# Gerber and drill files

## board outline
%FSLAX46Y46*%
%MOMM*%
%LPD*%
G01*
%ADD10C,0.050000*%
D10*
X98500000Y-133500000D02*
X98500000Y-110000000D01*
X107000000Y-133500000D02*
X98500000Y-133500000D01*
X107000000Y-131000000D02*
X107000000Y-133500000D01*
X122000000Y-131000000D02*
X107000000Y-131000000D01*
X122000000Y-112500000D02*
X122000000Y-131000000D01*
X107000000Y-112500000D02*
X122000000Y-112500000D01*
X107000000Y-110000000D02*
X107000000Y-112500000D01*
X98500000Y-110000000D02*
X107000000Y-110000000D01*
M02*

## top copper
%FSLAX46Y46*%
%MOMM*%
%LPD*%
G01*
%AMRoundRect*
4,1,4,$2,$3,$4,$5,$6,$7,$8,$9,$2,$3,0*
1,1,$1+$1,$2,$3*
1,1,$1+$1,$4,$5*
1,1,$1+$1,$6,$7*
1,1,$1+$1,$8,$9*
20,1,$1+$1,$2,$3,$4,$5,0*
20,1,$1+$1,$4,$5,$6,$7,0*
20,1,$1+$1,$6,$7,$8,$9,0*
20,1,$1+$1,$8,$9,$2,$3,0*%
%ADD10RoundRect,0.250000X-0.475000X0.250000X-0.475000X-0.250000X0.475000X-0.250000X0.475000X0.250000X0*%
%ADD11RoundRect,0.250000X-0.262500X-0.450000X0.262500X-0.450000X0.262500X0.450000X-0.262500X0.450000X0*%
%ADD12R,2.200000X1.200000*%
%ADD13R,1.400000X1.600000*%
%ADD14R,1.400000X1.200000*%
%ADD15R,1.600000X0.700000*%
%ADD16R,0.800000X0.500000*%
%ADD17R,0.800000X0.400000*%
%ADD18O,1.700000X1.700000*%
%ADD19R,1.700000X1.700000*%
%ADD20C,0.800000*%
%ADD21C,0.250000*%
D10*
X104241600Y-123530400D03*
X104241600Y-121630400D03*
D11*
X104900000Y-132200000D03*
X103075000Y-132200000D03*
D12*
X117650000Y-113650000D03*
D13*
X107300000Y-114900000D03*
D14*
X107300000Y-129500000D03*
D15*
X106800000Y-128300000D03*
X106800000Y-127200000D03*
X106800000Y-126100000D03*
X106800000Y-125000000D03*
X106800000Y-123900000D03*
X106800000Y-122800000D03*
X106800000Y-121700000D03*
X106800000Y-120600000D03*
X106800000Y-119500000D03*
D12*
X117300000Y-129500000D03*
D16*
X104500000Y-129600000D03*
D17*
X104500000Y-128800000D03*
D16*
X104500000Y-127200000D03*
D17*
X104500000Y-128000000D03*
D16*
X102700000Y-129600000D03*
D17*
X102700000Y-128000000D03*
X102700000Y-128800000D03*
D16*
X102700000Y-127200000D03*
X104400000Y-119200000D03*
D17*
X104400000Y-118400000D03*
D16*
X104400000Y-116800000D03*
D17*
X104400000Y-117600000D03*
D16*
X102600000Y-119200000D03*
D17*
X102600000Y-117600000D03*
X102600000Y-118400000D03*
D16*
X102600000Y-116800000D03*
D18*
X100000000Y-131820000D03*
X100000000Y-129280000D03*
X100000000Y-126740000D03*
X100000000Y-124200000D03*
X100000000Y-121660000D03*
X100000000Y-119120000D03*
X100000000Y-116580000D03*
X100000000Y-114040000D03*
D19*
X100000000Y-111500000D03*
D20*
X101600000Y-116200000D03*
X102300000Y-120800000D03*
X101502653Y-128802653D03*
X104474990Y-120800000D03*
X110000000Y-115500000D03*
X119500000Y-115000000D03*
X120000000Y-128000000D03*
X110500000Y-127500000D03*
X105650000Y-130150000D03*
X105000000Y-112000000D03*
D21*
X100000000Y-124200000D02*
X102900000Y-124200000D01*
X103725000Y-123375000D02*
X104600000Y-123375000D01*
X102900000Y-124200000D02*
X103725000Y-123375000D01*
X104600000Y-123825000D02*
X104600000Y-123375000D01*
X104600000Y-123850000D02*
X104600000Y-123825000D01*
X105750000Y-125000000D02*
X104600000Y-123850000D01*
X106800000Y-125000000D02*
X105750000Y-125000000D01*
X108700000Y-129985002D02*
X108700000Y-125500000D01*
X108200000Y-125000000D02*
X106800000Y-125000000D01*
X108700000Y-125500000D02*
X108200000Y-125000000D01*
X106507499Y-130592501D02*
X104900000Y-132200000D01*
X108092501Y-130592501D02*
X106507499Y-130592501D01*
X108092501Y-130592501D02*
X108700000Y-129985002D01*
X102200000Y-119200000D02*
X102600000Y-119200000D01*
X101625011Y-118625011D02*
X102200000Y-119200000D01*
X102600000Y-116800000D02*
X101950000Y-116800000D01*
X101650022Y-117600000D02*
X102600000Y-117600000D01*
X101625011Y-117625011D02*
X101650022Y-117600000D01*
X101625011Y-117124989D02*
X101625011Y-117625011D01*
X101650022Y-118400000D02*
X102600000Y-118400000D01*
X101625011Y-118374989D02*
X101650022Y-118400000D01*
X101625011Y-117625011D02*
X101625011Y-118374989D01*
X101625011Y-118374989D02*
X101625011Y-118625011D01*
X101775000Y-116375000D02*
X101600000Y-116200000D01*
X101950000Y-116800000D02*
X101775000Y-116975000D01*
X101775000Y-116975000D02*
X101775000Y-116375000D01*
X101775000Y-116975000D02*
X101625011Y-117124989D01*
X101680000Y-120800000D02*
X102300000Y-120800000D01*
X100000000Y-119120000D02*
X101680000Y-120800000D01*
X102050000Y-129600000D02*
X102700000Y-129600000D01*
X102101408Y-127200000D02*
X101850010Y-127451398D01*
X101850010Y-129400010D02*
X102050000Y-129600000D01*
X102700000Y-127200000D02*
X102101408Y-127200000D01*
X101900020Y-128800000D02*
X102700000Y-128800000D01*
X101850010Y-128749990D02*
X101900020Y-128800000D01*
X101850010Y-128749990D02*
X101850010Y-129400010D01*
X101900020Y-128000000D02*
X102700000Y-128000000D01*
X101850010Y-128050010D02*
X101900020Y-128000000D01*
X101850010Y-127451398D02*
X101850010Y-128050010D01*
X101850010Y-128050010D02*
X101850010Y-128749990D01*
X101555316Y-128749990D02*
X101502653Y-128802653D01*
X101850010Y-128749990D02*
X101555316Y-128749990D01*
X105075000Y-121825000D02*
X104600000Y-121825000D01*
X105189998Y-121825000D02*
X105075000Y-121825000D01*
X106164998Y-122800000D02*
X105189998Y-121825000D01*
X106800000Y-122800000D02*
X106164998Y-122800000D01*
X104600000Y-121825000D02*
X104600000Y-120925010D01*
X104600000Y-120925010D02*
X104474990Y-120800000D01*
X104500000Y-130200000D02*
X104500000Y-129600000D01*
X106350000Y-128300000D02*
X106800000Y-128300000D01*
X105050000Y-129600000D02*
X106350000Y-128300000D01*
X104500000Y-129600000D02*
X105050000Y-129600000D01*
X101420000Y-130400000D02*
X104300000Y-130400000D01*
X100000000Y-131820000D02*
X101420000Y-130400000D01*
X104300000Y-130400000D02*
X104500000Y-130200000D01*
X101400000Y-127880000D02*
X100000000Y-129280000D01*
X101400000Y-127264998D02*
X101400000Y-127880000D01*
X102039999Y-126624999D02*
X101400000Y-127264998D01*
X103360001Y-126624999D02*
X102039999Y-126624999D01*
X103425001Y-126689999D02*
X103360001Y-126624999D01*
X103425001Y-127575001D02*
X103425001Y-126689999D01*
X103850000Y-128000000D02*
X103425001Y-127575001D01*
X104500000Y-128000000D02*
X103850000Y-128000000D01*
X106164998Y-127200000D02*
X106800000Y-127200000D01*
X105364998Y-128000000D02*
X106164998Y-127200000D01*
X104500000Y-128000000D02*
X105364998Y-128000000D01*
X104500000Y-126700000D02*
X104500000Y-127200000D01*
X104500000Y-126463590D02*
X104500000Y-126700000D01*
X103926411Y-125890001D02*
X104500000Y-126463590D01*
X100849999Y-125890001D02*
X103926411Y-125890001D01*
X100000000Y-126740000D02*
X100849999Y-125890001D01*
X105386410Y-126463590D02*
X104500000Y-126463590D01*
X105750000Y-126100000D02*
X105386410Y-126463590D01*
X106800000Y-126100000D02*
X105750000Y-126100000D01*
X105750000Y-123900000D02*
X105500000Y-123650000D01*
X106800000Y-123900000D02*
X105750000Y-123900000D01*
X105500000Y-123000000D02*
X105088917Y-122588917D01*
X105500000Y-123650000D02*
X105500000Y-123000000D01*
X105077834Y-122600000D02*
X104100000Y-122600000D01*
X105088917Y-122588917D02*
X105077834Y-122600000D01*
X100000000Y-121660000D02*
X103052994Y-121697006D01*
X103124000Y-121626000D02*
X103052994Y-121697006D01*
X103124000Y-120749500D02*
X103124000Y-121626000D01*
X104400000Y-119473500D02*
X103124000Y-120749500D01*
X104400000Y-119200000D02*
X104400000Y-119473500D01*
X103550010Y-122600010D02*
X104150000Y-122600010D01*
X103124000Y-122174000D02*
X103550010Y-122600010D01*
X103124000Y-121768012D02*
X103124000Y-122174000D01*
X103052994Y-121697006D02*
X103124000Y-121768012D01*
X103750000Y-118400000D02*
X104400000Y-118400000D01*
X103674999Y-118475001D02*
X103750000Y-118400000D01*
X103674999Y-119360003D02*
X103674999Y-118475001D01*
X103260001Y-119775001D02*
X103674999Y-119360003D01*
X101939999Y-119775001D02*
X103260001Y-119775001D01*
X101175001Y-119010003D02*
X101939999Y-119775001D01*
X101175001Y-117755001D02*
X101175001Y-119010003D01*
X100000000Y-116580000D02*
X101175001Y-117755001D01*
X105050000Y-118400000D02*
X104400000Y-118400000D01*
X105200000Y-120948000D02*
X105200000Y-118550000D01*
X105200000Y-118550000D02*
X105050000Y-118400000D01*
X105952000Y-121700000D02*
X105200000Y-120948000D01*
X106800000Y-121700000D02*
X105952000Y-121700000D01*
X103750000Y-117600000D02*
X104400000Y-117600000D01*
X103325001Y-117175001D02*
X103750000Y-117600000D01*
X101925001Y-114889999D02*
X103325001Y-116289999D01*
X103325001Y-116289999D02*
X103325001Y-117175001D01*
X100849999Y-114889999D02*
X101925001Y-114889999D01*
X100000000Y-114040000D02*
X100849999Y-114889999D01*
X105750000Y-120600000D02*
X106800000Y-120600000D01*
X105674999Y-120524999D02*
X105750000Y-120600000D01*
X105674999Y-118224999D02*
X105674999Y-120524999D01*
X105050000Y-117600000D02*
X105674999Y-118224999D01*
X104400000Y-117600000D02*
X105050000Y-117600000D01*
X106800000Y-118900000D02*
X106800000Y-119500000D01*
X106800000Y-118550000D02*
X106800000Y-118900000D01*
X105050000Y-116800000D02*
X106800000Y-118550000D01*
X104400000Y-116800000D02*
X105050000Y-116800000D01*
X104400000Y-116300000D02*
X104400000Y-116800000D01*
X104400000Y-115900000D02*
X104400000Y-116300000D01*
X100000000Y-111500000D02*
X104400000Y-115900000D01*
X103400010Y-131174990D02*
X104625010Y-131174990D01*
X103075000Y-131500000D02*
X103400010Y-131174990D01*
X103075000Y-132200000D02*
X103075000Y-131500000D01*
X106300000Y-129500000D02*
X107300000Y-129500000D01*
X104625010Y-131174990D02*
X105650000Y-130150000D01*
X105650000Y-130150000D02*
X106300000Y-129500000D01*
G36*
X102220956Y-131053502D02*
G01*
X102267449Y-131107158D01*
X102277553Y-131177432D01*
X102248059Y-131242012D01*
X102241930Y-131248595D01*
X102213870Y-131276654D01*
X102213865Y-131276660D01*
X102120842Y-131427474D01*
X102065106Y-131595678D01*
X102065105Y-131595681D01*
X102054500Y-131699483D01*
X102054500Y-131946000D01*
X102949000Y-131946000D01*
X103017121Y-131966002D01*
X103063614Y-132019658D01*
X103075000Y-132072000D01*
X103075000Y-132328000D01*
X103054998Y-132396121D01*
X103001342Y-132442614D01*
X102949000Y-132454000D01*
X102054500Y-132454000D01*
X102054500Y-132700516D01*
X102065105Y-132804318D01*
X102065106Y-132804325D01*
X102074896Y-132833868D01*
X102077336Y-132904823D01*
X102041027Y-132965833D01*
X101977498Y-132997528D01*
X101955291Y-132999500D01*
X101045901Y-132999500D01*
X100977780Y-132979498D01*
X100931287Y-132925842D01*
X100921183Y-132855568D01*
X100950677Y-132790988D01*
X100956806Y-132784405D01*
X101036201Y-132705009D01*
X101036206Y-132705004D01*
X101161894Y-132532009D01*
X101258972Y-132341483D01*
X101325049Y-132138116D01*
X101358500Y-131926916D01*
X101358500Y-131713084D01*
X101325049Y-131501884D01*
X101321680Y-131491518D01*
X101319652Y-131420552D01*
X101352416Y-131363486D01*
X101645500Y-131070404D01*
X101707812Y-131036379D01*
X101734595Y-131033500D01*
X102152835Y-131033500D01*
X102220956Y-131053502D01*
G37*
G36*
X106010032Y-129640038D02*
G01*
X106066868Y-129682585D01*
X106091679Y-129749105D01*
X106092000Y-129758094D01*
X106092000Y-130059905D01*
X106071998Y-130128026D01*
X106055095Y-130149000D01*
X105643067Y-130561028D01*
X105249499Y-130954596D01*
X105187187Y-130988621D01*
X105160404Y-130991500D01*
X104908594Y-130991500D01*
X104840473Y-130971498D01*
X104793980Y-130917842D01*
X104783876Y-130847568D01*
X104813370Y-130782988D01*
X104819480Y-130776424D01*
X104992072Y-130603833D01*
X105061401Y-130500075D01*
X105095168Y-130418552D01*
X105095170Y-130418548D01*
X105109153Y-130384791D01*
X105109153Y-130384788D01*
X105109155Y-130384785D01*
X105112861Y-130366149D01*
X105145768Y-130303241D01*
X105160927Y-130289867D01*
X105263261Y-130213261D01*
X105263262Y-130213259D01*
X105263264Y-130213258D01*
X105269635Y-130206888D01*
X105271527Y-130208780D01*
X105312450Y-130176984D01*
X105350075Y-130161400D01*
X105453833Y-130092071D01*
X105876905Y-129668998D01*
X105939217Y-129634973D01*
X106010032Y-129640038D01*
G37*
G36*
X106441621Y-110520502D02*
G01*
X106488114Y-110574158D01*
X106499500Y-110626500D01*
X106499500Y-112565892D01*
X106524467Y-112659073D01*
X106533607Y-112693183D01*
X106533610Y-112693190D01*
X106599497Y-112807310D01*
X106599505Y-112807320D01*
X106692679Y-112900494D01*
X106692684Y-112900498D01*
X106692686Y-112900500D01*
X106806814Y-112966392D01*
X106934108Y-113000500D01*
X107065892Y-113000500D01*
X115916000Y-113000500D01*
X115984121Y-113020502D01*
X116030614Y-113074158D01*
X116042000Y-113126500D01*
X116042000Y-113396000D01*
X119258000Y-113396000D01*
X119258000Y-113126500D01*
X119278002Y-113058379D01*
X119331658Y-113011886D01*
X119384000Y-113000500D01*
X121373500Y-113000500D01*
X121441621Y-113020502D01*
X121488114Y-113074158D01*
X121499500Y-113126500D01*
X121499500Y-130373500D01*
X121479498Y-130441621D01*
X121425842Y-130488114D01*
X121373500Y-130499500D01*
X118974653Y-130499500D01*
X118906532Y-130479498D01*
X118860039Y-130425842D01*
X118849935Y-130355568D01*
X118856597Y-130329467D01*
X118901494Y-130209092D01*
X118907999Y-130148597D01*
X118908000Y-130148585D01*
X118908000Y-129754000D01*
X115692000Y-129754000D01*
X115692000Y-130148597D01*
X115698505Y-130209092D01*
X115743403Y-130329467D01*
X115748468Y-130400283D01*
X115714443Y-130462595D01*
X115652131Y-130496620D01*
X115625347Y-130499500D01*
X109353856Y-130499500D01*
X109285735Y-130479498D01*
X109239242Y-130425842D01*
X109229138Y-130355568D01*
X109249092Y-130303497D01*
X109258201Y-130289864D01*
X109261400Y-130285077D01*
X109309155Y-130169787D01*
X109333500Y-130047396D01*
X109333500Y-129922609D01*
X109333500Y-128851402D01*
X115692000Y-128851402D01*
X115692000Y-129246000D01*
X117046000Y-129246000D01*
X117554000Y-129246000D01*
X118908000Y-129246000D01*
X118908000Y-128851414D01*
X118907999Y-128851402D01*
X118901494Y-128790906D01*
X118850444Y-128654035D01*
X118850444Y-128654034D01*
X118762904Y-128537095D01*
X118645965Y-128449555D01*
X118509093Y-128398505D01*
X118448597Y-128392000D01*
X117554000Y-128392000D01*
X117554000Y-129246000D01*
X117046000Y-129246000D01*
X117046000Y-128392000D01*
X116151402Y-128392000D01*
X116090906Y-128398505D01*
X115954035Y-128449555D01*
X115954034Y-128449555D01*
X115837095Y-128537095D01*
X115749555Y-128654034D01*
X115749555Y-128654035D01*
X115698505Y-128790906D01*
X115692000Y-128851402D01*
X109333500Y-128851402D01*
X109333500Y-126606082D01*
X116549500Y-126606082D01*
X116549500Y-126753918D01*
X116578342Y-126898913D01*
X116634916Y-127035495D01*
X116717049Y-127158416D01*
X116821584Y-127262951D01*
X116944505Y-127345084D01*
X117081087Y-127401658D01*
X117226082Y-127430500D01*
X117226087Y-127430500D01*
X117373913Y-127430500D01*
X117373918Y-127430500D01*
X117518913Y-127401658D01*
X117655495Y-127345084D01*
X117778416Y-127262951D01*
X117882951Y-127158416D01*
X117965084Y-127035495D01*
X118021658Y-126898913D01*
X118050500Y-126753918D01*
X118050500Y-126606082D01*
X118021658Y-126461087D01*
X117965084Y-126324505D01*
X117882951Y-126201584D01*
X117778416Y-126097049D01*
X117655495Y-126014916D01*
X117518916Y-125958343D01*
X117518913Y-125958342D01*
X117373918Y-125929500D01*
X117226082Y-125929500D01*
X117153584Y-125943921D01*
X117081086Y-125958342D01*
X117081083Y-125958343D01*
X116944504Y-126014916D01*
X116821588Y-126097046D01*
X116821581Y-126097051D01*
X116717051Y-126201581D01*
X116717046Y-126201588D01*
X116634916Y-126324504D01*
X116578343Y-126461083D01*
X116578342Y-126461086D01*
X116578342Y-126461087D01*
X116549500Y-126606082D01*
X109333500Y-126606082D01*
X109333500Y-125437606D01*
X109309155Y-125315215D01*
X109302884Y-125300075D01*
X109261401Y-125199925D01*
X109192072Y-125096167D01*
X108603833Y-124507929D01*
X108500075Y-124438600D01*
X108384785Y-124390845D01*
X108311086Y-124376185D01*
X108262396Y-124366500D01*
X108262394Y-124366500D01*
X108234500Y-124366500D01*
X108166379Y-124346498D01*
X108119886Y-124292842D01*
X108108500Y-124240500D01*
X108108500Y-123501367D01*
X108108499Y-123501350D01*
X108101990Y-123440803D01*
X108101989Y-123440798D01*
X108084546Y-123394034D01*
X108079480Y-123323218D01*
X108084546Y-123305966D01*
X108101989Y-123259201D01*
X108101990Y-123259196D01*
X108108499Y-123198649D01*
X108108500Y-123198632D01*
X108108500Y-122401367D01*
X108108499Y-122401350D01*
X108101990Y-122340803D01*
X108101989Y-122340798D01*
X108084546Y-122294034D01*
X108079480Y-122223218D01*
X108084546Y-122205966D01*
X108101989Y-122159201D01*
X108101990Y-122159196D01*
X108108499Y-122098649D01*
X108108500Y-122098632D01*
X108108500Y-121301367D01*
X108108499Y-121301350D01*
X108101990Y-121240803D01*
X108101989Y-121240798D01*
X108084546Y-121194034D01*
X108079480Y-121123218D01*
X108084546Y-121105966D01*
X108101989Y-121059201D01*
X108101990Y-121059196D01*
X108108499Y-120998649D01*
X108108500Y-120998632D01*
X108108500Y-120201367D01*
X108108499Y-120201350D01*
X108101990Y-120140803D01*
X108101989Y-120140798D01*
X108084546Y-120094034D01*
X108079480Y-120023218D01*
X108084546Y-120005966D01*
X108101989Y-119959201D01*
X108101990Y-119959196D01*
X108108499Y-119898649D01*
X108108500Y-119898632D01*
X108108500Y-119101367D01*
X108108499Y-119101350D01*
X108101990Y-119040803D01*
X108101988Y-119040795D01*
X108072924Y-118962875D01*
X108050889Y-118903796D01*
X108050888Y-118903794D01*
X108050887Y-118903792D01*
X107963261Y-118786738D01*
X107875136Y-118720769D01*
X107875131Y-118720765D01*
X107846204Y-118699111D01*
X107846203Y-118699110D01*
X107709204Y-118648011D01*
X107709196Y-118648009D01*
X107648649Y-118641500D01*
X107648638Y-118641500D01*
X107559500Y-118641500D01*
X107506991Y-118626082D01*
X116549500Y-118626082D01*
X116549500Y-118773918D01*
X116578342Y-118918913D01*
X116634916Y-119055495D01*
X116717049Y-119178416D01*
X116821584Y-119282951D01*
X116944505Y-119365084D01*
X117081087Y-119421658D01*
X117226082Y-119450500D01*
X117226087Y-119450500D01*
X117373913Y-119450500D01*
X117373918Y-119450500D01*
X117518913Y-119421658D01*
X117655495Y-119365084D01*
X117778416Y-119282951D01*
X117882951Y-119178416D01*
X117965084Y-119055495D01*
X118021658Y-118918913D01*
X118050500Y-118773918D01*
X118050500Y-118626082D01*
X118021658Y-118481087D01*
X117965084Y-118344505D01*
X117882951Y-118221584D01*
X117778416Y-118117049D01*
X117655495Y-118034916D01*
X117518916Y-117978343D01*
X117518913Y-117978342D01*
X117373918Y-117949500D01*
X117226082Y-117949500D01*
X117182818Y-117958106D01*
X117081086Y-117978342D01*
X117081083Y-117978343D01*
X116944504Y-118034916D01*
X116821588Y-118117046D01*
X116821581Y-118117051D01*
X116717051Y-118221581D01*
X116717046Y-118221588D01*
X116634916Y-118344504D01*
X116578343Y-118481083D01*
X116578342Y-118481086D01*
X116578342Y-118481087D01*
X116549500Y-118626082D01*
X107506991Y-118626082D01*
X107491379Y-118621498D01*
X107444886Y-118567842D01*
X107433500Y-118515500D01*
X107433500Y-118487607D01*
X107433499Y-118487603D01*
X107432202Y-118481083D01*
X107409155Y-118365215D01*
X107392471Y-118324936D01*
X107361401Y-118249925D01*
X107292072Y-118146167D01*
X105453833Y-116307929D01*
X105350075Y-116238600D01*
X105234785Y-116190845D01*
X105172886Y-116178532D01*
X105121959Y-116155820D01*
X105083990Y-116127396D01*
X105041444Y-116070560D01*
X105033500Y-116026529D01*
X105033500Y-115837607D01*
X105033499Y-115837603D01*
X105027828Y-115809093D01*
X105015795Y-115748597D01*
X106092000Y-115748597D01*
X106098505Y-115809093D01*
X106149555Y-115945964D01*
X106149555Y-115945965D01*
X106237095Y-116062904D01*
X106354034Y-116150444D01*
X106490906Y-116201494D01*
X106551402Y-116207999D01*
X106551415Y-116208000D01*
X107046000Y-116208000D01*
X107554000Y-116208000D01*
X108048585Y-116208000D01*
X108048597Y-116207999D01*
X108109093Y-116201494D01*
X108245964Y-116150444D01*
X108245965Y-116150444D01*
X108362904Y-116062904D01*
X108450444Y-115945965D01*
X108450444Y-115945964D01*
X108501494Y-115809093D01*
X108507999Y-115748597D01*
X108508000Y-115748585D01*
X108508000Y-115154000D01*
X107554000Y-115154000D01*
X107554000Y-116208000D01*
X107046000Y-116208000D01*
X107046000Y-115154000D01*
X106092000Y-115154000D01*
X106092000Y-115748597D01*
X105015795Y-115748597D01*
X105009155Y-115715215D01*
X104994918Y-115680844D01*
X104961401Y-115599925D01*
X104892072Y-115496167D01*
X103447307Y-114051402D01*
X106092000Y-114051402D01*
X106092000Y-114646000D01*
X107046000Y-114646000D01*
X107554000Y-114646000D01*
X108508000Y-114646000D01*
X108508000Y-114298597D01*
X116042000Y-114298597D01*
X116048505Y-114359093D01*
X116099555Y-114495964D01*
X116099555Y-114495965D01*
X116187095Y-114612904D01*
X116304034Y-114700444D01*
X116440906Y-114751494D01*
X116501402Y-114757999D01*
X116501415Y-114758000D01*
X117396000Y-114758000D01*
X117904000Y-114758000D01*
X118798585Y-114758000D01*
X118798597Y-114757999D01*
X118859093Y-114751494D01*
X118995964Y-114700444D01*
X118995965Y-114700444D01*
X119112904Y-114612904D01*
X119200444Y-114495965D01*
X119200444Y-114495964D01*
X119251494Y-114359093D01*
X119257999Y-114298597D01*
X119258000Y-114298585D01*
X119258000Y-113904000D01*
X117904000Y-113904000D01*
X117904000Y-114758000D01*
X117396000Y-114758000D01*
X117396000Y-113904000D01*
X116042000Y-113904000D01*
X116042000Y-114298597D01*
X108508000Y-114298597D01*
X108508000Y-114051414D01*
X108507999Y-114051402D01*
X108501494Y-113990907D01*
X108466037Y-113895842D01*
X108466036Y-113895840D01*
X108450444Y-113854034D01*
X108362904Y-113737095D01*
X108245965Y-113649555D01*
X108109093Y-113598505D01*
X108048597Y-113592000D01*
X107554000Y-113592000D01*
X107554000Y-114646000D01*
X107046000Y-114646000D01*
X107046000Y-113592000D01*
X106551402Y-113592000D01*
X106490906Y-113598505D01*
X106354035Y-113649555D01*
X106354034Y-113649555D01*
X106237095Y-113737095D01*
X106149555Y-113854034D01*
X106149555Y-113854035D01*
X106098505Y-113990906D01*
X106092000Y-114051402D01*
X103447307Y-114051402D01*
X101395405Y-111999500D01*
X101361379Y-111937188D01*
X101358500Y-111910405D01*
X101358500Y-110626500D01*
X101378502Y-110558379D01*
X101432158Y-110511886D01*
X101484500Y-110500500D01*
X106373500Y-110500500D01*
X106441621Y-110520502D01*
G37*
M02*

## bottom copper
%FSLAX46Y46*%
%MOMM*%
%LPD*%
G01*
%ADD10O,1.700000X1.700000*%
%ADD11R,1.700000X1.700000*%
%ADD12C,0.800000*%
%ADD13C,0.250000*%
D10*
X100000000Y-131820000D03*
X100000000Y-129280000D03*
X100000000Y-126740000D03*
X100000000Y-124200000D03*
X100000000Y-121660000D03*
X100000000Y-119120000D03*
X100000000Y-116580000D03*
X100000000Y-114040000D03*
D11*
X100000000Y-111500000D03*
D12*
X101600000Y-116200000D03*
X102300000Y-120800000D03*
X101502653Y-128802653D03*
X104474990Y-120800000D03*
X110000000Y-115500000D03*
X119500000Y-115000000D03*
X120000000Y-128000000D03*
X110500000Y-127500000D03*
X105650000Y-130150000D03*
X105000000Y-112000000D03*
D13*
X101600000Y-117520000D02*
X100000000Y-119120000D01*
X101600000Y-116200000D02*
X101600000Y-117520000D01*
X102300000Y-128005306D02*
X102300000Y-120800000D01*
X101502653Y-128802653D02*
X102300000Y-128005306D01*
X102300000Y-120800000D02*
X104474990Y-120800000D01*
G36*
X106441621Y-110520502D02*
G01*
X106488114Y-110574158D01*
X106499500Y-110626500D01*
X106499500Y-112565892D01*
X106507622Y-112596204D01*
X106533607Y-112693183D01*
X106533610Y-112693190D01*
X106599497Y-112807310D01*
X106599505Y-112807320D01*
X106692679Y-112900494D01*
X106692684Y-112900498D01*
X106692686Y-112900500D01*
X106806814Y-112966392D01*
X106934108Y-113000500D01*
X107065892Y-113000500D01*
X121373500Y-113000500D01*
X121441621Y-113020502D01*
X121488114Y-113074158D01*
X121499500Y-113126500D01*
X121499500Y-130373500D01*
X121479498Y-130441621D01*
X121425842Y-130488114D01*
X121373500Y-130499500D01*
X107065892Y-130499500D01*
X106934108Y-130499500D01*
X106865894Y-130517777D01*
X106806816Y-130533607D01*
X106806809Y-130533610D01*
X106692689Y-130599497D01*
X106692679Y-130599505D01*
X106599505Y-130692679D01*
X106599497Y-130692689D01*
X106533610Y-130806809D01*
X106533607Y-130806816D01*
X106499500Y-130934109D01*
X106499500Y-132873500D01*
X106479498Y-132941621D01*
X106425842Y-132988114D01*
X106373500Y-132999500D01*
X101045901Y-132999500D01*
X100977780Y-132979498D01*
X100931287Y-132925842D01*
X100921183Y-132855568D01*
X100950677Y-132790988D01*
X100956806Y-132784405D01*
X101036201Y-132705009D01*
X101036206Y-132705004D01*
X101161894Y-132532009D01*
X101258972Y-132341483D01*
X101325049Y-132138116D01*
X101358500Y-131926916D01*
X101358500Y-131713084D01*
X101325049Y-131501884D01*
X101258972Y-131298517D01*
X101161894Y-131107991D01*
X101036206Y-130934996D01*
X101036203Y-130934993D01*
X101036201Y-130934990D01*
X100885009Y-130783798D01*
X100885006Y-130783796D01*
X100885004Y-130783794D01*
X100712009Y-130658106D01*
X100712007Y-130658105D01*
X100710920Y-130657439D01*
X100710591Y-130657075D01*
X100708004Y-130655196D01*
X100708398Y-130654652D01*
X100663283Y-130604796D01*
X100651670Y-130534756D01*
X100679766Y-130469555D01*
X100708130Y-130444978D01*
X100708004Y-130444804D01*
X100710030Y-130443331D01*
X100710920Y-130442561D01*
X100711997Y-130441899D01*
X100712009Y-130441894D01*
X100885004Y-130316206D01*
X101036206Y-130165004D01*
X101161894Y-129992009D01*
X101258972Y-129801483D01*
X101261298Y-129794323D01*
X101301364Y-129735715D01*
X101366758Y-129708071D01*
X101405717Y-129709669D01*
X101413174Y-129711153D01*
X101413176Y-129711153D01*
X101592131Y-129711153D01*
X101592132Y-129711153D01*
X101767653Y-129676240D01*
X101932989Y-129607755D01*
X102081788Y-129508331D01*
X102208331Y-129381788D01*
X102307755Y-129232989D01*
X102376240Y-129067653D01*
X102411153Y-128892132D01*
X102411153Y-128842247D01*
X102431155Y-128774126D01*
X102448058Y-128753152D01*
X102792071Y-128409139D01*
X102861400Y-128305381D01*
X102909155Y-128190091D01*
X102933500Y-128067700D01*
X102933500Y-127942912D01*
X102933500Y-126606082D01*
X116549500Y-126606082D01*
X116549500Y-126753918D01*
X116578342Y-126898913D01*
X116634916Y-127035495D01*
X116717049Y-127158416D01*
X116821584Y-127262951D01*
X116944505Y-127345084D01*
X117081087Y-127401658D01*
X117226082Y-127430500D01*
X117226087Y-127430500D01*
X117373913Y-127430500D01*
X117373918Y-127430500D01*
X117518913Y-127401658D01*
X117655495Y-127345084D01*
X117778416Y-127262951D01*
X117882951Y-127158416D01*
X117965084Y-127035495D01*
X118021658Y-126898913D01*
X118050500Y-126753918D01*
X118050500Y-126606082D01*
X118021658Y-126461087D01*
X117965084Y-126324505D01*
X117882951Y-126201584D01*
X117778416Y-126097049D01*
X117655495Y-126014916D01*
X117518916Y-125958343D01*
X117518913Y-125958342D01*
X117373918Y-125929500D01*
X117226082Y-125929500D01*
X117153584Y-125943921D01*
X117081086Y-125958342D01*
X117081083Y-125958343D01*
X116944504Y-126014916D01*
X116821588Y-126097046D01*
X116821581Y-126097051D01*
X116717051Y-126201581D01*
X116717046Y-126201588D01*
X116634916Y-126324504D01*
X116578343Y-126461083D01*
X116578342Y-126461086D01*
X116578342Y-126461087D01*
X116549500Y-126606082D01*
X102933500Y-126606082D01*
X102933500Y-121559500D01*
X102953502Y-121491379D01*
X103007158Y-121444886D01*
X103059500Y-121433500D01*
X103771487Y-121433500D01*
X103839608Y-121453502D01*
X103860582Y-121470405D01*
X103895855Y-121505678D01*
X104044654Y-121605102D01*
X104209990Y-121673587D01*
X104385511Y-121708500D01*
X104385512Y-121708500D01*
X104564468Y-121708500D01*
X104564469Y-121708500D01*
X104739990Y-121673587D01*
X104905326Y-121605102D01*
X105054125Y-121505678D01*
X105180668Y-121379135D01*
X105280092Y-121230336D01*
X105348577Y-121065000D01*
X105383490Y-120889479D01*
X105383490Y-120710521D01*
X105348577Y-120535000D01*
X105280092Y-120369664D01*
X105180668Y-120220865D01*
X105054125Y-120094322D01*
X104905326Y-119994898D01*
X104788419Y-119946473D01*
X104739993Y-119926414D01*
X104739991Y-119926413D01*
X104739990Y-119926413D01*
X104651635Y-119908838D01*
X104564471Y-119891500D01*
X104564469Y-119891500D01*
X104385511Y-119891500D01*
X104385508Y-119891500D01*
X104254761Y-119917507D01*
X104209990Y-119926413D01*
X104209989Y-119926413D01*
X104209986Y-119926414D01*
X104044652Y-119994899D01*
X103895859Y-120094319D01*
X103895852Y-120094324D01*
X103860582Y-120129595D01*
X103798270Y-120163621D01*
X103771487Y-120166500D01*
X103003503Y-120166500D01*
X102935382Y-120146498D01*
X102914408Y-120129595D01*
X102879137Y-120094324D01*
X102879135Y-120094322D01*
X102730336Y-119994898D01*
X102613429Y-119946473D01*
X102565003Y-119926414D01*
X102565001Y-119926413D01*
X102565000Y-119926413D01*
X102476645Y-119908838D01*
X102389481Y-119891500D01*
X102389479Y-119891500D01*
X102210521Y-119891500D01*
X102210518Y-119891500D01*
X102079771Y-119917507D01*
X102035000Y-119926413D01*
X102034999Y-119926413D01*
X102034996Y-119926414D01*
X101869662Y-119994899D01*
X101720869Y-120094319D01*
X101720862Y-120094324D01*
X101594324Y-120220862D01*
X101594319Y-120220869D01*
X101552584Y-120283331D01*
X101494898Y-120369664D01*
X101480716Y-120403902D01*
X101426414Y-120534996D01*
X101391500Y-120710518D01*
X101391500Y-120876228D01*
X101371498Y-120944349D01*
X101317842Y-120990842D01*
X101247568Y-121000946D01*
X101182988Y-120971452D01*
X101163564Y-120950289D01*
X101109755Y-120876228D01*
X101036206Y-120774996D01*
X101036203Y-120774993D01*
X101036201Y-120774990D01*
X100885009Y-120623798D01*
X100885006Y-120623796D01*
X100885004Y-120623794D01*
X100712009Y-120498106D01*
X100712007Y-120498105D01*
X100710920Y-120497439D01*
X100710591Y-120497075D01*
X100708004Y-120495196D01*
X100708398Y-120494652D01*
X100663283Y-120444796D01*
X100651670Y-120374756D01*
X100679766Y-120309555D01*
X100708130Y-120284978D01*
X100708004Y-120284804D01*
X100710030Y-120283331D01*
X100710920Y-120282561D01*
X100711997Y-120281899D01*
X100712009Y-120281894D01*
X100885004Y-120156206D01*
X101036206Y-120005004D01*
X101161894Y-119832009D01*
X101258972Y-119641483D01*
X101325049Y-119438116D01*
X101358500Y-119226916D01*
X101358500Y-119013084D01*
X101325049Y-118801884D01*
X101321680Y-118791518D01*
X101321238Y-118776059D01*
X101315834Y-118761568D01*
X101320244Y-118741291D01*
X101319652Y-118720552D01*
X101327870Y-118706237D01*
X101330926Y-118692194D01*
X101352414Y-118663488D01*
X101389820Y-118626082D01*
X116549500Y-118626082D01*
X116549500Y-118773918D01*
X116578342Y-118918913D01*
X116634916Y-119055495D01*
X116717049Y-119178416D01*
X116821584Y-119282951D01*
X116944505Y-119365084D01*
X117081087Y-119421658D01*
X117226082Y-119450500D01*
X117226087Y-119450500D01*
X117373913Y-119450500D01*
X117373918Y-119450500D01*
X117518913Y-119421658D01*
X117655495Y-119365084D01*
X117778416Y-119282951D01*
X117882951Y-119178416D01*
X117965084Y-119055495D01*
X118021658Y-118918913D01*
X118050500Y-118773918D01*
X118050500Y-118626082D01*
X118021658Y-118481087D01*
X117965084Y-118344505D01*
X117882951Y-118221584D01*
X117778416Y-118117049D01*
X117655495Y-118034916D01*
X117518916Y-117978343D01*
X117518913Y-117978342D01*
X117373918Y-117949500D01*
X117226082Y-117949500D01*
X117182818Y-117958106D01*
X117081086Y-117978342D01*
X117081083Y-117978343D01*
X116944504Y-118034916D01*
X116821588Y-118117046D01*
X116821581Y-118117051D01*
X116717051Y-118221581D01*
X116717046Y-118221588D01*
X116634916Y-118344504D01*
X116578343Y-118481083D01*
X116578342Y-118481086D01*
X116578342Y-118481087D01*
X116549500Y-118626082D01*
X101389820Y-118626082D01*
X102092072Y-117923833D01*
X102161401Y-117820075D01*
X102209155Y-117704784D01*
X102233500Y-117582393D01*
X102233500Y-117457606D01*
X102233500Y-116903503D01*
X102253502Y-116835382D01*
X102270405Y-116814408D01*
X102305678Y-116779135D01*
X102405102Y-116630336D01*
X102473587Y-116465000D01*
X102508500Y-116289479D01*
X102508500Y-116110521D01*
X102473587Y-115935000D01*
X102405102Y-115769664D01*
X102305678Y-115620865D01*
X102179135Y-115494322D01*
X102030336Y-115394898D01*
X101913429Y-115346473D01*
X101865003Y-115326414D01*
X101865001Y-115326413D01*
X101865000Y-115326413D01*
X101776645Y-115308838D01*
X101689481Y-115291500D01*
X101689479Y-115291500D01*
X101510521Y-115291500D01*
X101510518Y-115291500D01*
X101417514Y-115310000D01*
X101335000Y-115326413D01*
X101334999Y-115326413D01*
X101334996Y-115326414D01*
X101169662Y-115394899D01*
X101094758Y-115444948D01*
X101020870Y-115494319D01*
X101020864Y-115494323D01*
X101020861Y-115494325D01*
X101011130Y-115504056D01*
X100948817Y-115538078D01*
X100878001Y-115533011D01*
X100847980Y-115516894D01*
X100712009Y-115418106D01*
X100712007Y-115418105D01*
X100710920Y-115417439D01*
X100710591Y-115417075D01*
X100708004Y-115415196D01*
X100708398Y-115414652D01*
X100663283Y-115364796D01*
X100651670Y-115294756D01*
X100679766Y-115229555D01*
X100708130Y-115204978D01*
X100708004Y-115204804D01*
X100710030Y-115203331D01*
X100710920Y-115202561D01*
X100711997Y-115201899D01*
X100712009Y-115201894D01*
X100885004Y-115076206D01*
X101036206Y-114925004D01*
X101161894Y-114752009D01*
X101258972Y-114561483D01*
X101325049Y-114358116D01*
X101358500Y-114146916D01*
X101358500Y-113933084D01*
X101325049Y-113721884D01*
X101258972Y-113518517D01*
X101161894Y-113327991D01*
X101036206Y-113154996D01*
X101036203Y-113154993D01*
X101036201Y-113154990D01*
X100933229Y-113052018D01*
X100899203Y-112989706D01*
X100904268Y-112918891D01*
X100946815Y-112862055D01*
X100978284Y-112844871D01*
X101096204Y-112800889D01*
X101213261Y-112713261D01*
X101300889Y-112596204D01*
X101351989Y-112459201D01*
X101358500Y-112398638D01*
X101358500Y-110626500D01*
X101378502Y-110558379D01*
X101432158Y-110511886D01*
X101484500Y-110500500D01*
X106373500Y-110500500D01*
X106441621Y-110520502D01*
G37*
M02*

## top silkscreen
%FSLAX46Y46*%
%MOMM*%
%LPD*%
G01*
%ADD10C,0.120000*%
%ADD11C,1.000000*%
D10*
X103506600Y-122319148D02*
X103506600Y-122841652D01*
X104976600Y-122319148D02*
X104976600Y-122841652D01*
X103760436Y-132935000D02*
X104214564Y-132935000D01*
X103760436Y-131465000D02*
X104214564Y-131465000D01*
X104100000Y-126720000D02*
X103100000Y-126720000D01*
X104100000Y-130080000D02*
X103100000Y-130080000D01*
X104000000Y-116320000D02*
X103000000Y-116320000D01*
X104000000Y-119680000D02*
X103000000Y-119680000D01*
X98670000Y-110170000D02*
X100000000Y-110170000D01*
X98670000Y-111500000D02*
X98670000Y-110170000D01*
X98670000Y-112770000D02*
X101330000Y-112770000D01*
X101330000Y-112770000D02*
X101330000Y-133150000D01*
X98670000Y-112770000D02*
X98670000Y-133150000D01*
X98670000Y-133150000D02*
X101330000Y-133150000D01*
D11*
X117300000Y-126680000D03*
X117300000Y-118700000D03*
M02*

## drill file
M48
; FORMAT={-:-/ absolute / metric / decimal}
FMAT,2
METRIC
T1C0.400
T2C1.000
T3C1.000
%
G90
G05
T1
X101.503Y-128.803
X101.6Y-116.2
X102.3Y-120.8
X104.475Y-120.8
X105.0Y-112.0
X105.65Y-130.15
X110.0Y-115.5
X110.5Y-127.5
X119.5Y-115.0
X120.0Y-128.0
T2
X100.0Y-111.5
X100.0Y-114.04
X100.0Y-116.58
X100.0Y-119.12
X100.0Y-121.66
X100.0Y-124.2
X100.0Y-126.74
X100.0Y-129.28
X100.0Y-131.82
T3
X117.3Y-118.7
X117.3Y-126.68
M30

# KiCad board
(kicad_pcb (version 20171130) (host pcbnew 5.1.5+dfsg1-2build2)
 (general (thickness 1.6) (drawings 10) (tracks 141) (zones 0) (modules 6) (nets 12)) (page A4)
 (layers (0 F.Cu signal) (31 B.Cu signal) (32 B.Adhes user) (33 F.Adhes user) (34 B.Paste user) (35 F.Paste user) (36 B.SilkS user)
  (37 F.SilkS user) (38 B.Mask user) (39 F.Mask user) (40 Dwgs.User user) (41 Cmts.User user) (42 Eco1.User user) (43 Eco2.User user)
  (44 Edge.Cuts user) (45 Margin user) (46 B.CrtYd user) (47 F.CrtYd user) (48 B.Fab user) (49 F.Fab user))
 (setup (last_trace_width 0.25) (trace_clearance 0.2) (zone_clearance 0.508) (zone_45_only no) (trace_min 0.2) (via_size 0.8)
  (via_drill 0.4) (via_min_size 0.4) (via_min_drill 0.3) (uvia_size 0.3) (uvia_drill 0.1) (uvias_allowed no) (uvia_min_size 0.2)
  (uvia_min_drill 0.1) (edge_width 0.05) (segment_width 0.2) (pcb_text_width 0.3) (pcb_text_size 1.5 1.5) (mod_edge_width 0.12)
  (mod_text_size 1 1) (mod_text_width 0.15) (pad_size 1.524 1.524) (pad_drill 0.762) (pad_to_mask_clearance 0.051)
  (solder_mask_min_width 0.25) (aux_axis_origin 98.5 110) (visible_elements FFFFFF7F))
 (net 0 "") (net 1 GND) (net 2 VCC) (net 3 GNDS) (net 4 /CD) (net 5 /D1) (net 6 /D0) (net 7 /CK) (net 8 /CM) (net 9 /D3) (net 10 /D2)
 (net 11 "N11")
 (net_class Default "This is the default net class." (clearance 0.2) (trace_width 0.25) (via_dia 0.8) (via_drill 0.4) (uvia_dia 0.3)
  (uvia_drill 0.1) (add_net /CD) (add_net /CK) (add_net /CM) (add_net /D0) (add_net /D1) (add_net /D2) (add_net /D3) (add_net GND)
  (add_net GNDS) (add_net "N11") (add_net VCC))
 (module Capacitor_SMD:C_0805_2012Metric (layer F.Cu) (at 104.2416 122.5804 270)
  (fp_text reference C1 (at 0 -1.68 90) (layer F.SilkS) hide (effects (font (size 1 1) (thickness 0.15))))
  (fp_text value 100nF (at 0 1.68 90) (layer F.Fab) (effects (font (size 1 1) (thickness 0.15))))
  (fp_line (start -0.261252 0.735) (end 0.261252 0.735) (layer F.SilkS) (width 0.12))
  (fp_line (start -0.261252 -0.735) (end 0.261252 -0.735) (layer F.SilkS) (width 0.12))
  (pad 2 smd roundrect (at 0.95 0 270) (size 1 1.45) (layers F.Cu F.Paste F.Mask) (roundrect_rratio 0.25) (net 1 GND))
  (pad 1 smd roundrect (at -0.95 0 270) (size 1 1.45) (layers F.Cu F.Paste F.Mask) (roundrect_rratio 0.25) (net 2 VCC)))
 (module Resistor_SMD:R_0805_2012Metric (layer F.Cu) (at 103.9875 132.2)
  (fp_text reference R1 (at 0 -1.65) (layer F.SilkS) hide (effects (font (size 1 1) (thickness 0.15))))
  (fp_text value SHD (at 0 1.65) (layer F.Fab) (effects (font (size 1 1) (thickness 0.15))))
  (fp_line (start -0.227064 0.735) (end 0.227064 0.735) (layer F.SilkS) (width 0.12))
  (fp_line (start -0.227064 -0.735) (end 0.227064 -0.735) (layer F.SilkS) (width 0.12))
  (pad 2 smd roundrect (at 0.9125 0) (size 1.025 1.4) (layers F.Cu F.Paste F.Mask) (roundrect_rratio 0.243902) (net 1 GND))
  (pad 1 smd roundrect (at -0.9125 0) (size 1.025 1.4) (layers F.Cu F.Paste F.Mask) (roundrect_rratio 0.243902) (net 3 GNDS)))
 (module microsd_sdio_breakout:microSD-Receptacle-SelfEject (layer F.Cu) (at 106.8 121.75 90)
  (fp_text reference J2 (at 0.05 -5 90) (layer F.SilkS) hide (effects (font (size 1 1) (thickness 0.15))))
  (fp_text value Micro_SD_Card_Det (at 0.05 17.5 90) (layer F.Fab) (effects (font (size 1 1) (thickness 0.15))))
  (pad "" np_thru_hole circle (at -4.93 10.5 270) (size 1 1) (drill 1) (layers *.Cu *.Mask F.SilkS))
  (pad "" np_thru_hole circle (at 3.05 10.5 270) (size 1 1) (drill 1) (layers *.Cu *.Mask F.SilkS))
  (pad 11 smd rect (at 8.1 10.85 270) (size 1.2 2.2) (layers F.Cu F.Paste F.Mask) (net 3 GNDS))
  (pad 11 smd rect (at 6.85 0.5 270) (size 1.6 1.4) (layers F.Cu F.Paste F.Mask) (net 3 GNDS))
  (pad 11 smd rect (at -7.75 0.5 270) (size 1.2 1.4) (layers F.Cu F.Paste F.Mask) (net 3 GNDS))
  (pad 10 smd rect (at -6.55 0 270) (size 0.7 1.6) (layers F.Cu F.Paste F.Mask) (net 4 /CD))
  (pad 8 smd rect (at -5.45 0 270) (size 0.7 1.6) (layers F.Cu F.Paste F.Mask) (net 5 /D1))
  (pad 7 smd rect (at -4.35 0 270) (size 0.7 1.6) (layers F.Cu F.Paste F.Mask) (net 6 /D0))
  (pad 6 smd rect (at -3.25 0 270) (size 0.7 1.6) (layers F.Cu F.Paste F.Mask) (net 1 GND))
  (pad 5 smd rect (at -2.15 0 270) (size 0.7 1.6) (layers F.Cu F.Paste F.Mask) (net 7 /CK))
  (pad 4 smd rect (at -1.05 0 270) (size 0.7 1.6) (layers F.Cu F.Paste F.Mask) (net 2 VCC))
  (pad 3 smd rect (at 0.05 0 270) (size 0.7 1.6) (layers F.Cu F.Paste F.Mask) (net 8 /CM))
  (pad 2 smd rect (at 1.15 0 270) (size 0.7 1.6) (layers F.Cu F.Paste F.Mask) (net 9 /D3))
  (pad 1 smd rect (at 2.25 0 270) (size 0.7 1.6) (layers F.Cu F.Paste F.Mask) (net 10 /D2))
  (pad 11 smd rect (at -7.75 10.5 270) (size 1.2 2.2) (layers F.Cu F.Paste F.Mask) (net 3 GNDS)))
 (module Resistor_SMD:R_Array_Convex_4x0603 (layer F.Cu) (at 103.6 128.4)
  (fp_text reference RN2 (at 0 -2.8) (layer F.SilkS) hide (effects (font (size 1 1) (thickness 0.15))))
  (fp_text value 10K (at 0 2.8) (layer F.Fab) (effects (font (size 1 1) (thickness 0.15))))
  (fp_line (start 0.5 -1.68) (end -0.5 -1.68) (layer F.SilkS) (width 0.12))
  (fp_line (start 0.5 1.68) (end -0.5 1.68) (layer F.SilkS) (width 0.12))
  (pad 5 smd rect (at 0.9 1.2) (size 0.8 0.5) (layers F.Cu F.Paste F.Mask) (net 4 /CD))
  (pad 6 smd rect (at 0.9 0.4) (size 0.8 0.4) (layers F.Cu F.Paste F.Mask) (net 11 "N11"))
  (pad 8 smd rect (at 0.9 -1.2) (size 0.8 0.5) (layers F.Cu F.Paste F.Mask) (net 6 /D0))
  (pad 7 smd rect (at 0.9 -0.4) (size 0.8 0.4) (layers F.Cu F.Paste F.Mask) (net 5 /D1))
  (pad 4 smd rect (at -0.9 1.2) (size 0.8 0.5) (layers F.Cu F.Paste F.Mask) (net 2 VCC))
  (pad 2 smd rect (at -0.9 -0.4) (size 0.8 0.4) (layers F.Cu F.Paste F.Mask) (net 2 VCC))
  (pad 3 smd rect (at -0.9 0.4) (size 0.8 0.4) (layers F.Cu F.Paste F.Mask) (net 2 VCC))
  (pad 1 smd rect (at -0.9 -1.2) (size 0.8 0.5) (layers F.Cu F.Paste F.Mask) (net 2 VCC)))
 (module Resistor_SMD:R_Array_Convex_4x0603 (layer F.Cu) (at 103.5 118)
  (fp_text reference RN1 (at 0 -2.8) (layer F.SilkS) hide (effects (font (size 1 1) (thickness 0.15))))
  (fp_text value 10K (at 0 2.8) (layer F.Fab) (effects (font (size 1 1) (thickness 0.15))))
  (fp_line (start 0.5 -1.68) (end -0.5 -1.68) (layer F.SilkS) (width 0.12))
  (fp_line (start 0.5 1.68) (end -0.5 1.68) (layer F.SilkS) (width 0.12))
  (pad 5 smd rect (at 0.9 1.2) (size 0.8 0.5) (layers F.Cu F.Paste F.Mask) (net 7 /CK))
  (pad 6 smd rect (at 0.9 0.4) (size 0.8 0.4) (layers F.Cu F.Paste F.Mask) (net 8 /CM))
  (pad 8 smd rect (at 0.9 -1.2) (size 0.8 0.5) (layers F.Cu F.Paste F.Mask) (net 10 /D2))
  (pad 7 smd rect (at 0.9 -0.4) (size 0.8 0.4) (layers F.Cu F.Paste F.Mask) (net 9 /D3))
  (pad 4 smd rect (at -0.9 1.2) (size 0.8 0.5) (layers F.Cu F.Paste F.Mask) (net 2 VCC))
  (pad 2 smd rect (at -0.9 -0.4) (size 0.8 0.4) (layers F.Cu F.Paste F.Mask) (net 2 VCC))
  (pad 3 smd rect (at -0.9 0.4) (size 0.8 0.4) (layers F.Cu F.Paste F.Mask) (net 2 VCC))
  (pad 1 smd rect (at -0.9 -1.2) (size 0.8 0.5) (layers F.Cu F.Paste F.Mask) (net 2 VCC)))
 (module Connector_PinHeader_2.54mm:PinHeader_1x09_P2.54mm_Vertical (layer F.Cu) (at 100 111.5)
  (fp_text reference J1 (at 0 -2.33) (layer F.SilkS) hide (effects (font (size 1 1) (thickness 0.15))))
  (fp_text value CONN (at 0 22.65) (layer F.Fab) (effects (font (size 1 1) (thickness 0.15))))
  (fp_line (start -1.33 -1.33) (end 0 -1.33) (layer F.SilkS) (width 0.12))
  (fp_line (start -1.33 0) (end -1.33 -1.33) (layer F.SilkS) (width 0.12))
  (fp_line (start -1.33 1.27) (end 1.33 1.27) (layer F.SilkS) (width 0.12))
  (fp_line (start 1.33 1.27) (end 1.33 21.65) (layer F.SilkS) (width 0.12))
  (fp_line (start -1.33 1.27) (end -1.33 21.65) (layer F.SilkS) (width 0.12))
  (fp_line (start -1.33 21.65) (end 1.33 21.65) (layer F.SilkS) (width 0.12))
  (pad 9 thru_hole oval (at 0 20.32) (size 1.7 1.7) (drill 1) (layers *.Cu *.Mask) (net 4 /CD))
  (pad 8 thru_hole oval (at 0 17.78) (size 1.7 1.7) (drill 1) (layers *.Cu *.Mask) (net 5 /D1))
  (pad 7 thru_hole oval (at 0 15.24) (size 1.7 1.7) (drill 1) (layers *.Cu *.Mask) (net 6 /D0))
  (pad 6 thru_hole oval (at 0 12.7) (size 1.7 1.7) (drill 1) (layers *.Cu *.Mask) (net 1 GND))
  (pad 5 thru_hole oval (at 0 10.16) (size 1.7 1.7) (drill 1) (layers *.Cu *.Mask) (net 7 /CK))
  (pad 4 thru_hole oval (at 0 7.62) (size 1.7 1.7) (drill 1) (layers *.Cu *.Mask) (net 2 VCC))
  (pad 3 thru_hole oval (at 0 5.08) (size 1.7 1.7) (drill 1) (layers *.Cu *.Mask) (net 8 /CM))
  (pad 2 thru_hole oval (at 0 2.54) (size 1.7 1.7) (drill 1) (layers *.Cu *.Mask) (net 9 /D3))
  (pad 1 thru_hole rect (at 0 0) (size 1.7 1.7) (drill 1) (layers *.Cu *.Mask) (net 10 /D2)))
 (gr_line (start 98.5 133.5) (end 98.5 110) (layer Edge.Cuts) (width 0.05))
 (gr_line (start 107 133.5) (end 98.5 133.5) (layer Edge.Cuts) (width 0.05))
 (gr_line (start 107 131) (end 107 133.5) (layer Edge.Cuts) (width 0.05))
 (gr_line (start 122 131) (end 107 131) (layer Edge.Cuts) (width 0.05))
 (gr_line (start 122 112.5) (end 122 131) (layer Edge.Cuts) (width 0.05))
 (gr_line (start 107 112.5) (end 122 112.5) (layer Edge.Cuts) (width 0.05))
 (gr_line (start 107 110) (end 107 112.5) (layer Edge.Cuts) (width 0.05))
 (gr_line (start 98.5 110) (end 107 110) (layer Edge.Cuts) (width 0.05))
 (segment (start 100 124.2) (end 102.9 124.2) (width 0.25) (layer F.Cu) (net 1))
 (segment (start 103.725 123.375) (end 104.6 123.375) (width 0.25) (layer F.Cu) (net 1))
 (segment (start 102.9 124.2) (end 103.725 123.375) (width 0.25) (layer F.Cu) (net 1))
 (segment (start 104.6 123.825) (end 104.6 123.375) (width 0.25) (layer F.Cu) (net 1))
 (segment (start 104.6 123.85) (end 104.6 123.825) (width 0.25) (layer F.Cu) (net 1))
 (segment (start 105.75 125) (end 104.6 123.85) (width 0.25) (layer F.Cu) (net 1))
 (segment (start 106.8 125) (end 105.75 125) (width 0.25) (layer F.Cu) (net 1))
 (segment (start 108.7 129.985002) (end 108.7 125.5) (width 0.25) (layer F.Cu) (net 1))
 (segment (start 108.2 125) (end 106.8 125) (width 0.25) (layer F.Cu) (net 1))
 (segment (start 108.7 125.5) (end 108.2 125) (width 0.25) (layer F.Cu) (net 1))
 (segment (start 106.507499 130.592501) (end 104.9 132.2) (width 0.25) (layer F.Cu) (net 1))
 (segment (start 108.092501 130.592501) (end 106.507499 130.592501) (width 0.25) (layer F.Cu) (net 1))
 (segment (start 108.092501 130.592501) (end 108.7 129.985002) (width 0.25) (layer F.Cu) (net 1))
 (segment (start 102.2 119.2) (end 102.6 119.2) (width 0.25) (layer F.Cu) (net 2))
 (segment (start 101.625011 118.625011) (end 102.2 119.2) (width 0.25) (layer F.Cu) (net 2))
 (segment (start 102.6 116.8) (end 101.95 116.8) (width 0.25) (layer F.Cu) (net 2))
 (segment (start 101.650022 117.6) (end 102.6 117.6) (width 0.25) (layer F.Cu) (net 2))
 (segment (start 101.625011 117.625011) (end 101.650022 117.6) (width 0.25) (layer F.Cu) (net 2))
 (segment (start 101.625011 117.124989) (end 101.625011 117.625011) (width 0.25) (layer F.Cu) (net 2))
 (segment (start 101.650022 118.4) (end 102.6 118.4) (width 0.25) (layer F.Cu) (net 2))
 (segment (start 101.625011 118.374989) (end 101.650022 118.4) (width 0.25) (layer F.Cu) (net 2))
 (segment (start 101.625011 117.625011) (end 101.625011 118.374989) (width 0.25) (layer F.Cu) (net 2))
 (segment (start 101.625011 118.374989) (end 101.625011 118.625011) (width 0.25) (layer F.Cu) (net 2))
 (via (at 101.6 116.2) (size 0.8) (drill 0.4) (layers F.Cu B.Cu) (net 2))
 (segment (start 101.775 116.375) (end 101.6 116.2) (width 0.25) (layer F.Cu) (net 2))
 (segment (start 101.95 116.8) (end 101.775 116.975) (width 0.25) (layer F.Cu) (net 2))
 (segment (start 101.775 116.975) (end 101.775 116.375) (width 0.25) (layer F.Cu) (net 2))
 (segment (start 101.775 116.975) (end 101.625011 117.124989) (width 0.25) (layer F.Cu) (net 2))
 (segment (start 101.6 117.52) (end 100 119.12) (width 0.25) (layer B.Cu) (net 2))
 (segment (start 101.6 116.2) (end 101.6 117.52) (width 0.25) (layer B.Cu) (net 2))
 (via (at 102.3 120.8) (size 0.8) (drill 0.4) (layers F.Cu B.Cu) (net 2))
 (segment (start 101.68 120.8) (end 102.3 120.8) (width 0.25) (layer F.Cu) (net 2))
 (segment (start 100 119.12) (end 101.68 120.8) (width 0.25) (layer F.Cu) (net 2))
 (segment (start 102.05 129.6) (end 102.7 129.6) (width 0.25) (layer F.Cu) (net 2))
 (segment (start 102.101408 127.2) (end 101.85001 127.451398) (width 0.25) (layer F.Cu) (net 2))
 (segment (start 101.85001 129.40001) (end 102.05 129.6) (width 0.25) (layer F.Cu) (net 2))
 (segment (start 102.7 127.2) (end 102.101408 127.2) (width 0.25) (layer F.Cu) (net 2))
 (segment (start 101.90002 128.8) (end 102.7 128.8) (width 0.25) (layer F.Cu) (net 2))
 (segment (start 101.85001 128.74999) (end 101.90002 128.8) (width 0.25) (layer F.Cu) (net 2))
 (segment (start 101.85001 128.74999) (end 101.85001 129.40001) (width 0.25) (layer F.Cu) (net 2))
 (segment (start 101.90002 128) (end 102.7 128) (width 0.25) (layer F.Cu) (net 2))
 (segment (start 101.85001 128.05001) (end 101.90002 128) (width 0.25) (layer F.Cu) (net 2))
 (segment (start 101.85001 127.451398) (end 101.85001 128.05001) (width 0.25) (layer F.Cu) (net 2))
 (segment (start 101.85001 128.05001) (end 101.85001 128.74999) (width 0.25) (layer F.Cu) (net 2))
 (via (at 101.502653 128.802653) (size 0.8) (drill 0.4) (layers F.Cu B.Cu) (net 2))
 (segment (start 101.555316 128.74999) (end 101.502653 128.802653) (width 0.25) (layer F.Cu) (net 2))
 (segment (start 101.85001 128.74999) (end 101.555316 128.74999) (width 0.25) (layer F.Cu) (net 2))
 (segment (start 102.3 128.005306) (end 102.3 120.8) (width 0.25) (layer B.Cu) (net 2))
 (segment (start 101.502653 128.802653) (end 102.3 128.005306) (width 0.25) (layer B.Cu) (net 2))
 (segment (start 105.075 121.825) (end 104.6 121.825) (width 0.25) (layer F.Cu) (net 2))
 (segment (start 105.189998 121.825) (end 105.075 121.825) (width 0.25) (layer F.Cu) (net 2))
 (segment (start 106.164998 122.8) (end 105.189998 121.825) (width 0.25) (layer F.Cu) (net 2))
 (segment (start 106.8 122.8) (end 106.164998 122.8) (width 0.25) (layer F.Cu) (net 2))
 (via (at 104.47499 120.8) (size 0.8) (drill 0.4) (layers F.Cu B.Cu) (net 2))
 (segment (start 102.3 120.8) (end 104.47499 120.8) (width 0.25) (layer B.Cu) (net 2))
 (segment (start 104.6 121.825) (end 104.6 120.92501) (width 0.25) (layer F.Cu) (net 2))
 (segment (start 104.6 120.92501) (end 104.47499 120.8) (width 0.25) (layer F.Cu) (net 2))
 (segment (start 104.5 130.2) (end 104.5 129.6) (width 0.25) (layer F.Cu) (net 4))
 (segment (start 106.35 128.3) (end 106.8 128.3) (width 0.25) (layer F.Cu) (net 4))
 (segment (start 105.05 129.6) (end 106.35 128.3) (width 0.25) (layer F.Cu) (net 4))
 (segment (start 104.5 129.6) (end 105.05 129.6) (width 0.25) (layer F.Cu) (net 4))
 (segment (start 101.42 130.4) (end 104.3 130.4) (width 0.25) (layer F.Cu) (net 4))
 (segment (start 100 131.82) (end 101.42 130.4) (width 0.25) (layer F.Cu) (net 4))
 (segment (start 104.3 130.4) (end 104.5 130.2) (width 0.25) (layer F.Cu) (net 4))
 (segment (start 101.4 127.88) (end 100 129.28) (width 0.25) (layer F.Cu) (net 5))
 (segment (start 101.4 127.264998) (end 101.4 127.88) (width 0.25) (layer F.Cu) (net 5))
 (segment (start 102.039999 126.624999) (end 101.4 127.264998) (width 0.25) (layer F.Cu) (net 5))
 (segment (start 103.360001 126.624999) (end 102.039999 126.624999) (width 0.25) (layer F.Cu) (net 5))
 (segment (start 103.425001 126.689999) (end 103.360001 126.624999) (width 0.25) (layer F.Cu) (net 5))
 (segment (start 103.425001 127.575001) (end 103.425001 126.689999) (width 0.25) (layer F.Cu) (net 5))
 (segment (start 103.85 128) (end 103.425001 127.575001) (width 0.25) (layer F.Cu) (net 5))
 (segment (start 104.5 128) (end 103.85 128) (width 0.25) (layer F.Cu) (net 5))
 (segment (start 106.164998 127.2) (end 106.8 127.2) (width 0.25) (layer F.Cu) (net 5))
 (segment (start 105.364998 128) (end 106.164998 127.2) (width 0.25) (layer F.Cu) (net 5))
 (segment (start 104.5 128) (end 105.364998 128) (width 0.25) (layer F.Cu) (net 5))
 (segment (start 104.5 126.7) (end 104.5 127.2) (width 0.25) (layer F.Cu) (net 6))
 (segment (start 104.5 126.46359) (end 104.5 126.7) (width 0.25) (layer F.Cu) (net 6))
 (segment (start 103.926411 125.890001) (end 104.5 126.46359) (width 0.25) (layer F.Cu) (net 6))
 (segment (start 100.849999 125.890001) (end 103.926411 125.890001) (width 0.25) (layer F.Cu) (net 6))
 (segment (start 100 126.74) (end 100.849999 125.890001) (width 0.25) (layer F.Cu) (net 6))
 (segment (start 105.38641 126.46359) (end 104.5 126.46359) (width 0.25) (layer F.Cu) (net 6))
 (segment (start 105.75 126.1) (end 105.38641 126.46359) (width 0.25) (layer F.Cu) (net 6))
 (segment (start 106.8 126.1) (end 105.75 126.1) (width 0.25) (layer F.Cu) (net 6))
 (segment (start 105.75 123.9) (end 105.5 123.65) (width 0.25) (layer F.Cu) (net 7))
 (segment (start 106.8 123.9) (end 105.75 123.9) (width 0.25) (layer F.Cu) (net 7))
 (segment (start 105.5 123) (end 105.088917 122.588917) (width 0.25) (layer F.Cu) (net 7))
 (segment (start 105.5 123.65) (end 105.5 123) (width 0.25) (layer F.Cu) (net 7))
 (segment (start 105.077834 122.6) (end 104.1 122.6) (width 0.25) (layer F.Cu) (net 7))
 (segment (start 105.088917 122.588917) (end 105.077834 122.6) (width 0.25) (layer F.Cu) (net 7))
 (segment (start 100 121.66) (end 103.052994 121.697006) (width 0.25) (layer F.Cu) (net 7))
 (segment (start 103.124 121.626) (end 103.052994 121.697006) (width 0.25) (layer F.Cu) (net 7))
 (segment (start 103.124 120.7495) (end 103.124 121.626) (width 0.25) (layer F.Cu) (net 7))
 (segment (start 104.4 119.4735) (end 103.124 120.7495) (width 0.25) (layer F.Cu) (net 7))
 (segment (start 104.4 119.2) (end 104.4 119.4735) (width 0.25) (layer F.Cu) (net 7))
 (segment (start 103.55001 122.60001) (end 104.15 122.60001) (width 0.25) (layer F.Cu) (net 7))
 (segment (start 103.124 122.174) (end 103.55001 122.60001) (width 0.25) (layer F.Cu) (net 7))
 (segment (start 103.124 121.768012) (end 103.124 122.174) (width 0.25) (layer F.Cu) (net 7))
 (segment (start 103.052994 121.697006) (end 103.124 121.768012) (width 0.25) (layer F.Cu) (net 7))
 (segment (start 103.75 118.4) (end 104.4 118.4) (width 0.25) (layer F.Cu) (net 8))
 (segment (start 103.674999 118.475001) (end 103.75 118.4) (width 0.25) (layer F.Cu) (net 8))
 (segment (start 103.674999 119.360003) (end 103.674999 118.475001) (width 0.25) (layer F.Cu) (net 8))
 (segment (start 103.260001 119.775001) (end 103.674999 119.360003) (width 0.25) (layer F.Cu) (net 8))
 (segment (start 101.939999 119.775001) (end 103.260001 119.775001) (width 0.25) (layer F.Cu) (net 8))
 (segment (start 101.175001 119.010003) (end 101.939999 119.775001) (width 0.25) (layer F.Cu) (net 8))
 (segment (start 101.175001 117.755001) (end 101.175001 119.010003) (width 0.25) (layer F.Cu) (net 8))
 (segment (start 100 116.58) (end 101.175001 117.755001) (width 0.25) (layer F.Cu) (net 8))
 (segment (start 105.05 118.4) (end 104.4 118.4) (width 0.25) (layer F.Cu) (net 8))
 (segment (start 105.2 120.948) (end 105.2 118.55) (width 0.25) (layer F.Cu) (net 8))
 (segment (start 105.2 118.55) (end 105.05 118.4) (width 0.25) (layer F.Cu) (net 8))
 (segment (start 105.952 121.7) (end 105.2 120.948) (width 0.25) (layer F.Cu) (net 8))
 (segment (start 106.8 121.7) (end 105.952 121.7) (width 0.25) (layer F.Cu) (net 8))
 (segment (start 103.75 117.6) (end 104.4 117.6) (width 0.25) (layer F.Cu) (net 9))
 (segment (start 103.325001 117.175001) (end 103.75 117.6) (width 0.25) (layer F.Cu) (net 9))
 (segment (start 101.925001 114.889999) (end 103.325001 116.289999) (width 0.25) (layer F.Cu) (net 9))
 (segment (start 103.325001 116.289999) (end 103.325001 117.175001) (width 0.25) (layer F.Cu) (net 9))
 (segment (start 100.849999 114.889999) (end 101.925001 114.889999) (width 0.25) (layer F.Cu) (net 9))
 (segment (start 100 114.04) (end 100.849999 114.889999) (width 0.25) (layer F.Cu) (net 9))
 (segment (start 105.75 120.6) (end 106.8 120.6) (width 0.25) (layer F.Cu) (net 9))
 (segment (start 105.674999 120.524999) (end 105.75 120.6) (width 0.25) (layer F.Cu) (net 9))
 (segment (start 105.674999 118.224999) (end 105.674999 120.524999) (width 0.25) (layer F.Cu) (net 9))
 (segment (start 105.05 117.6) (end 105.674999 118.224999) (width 0.25) (layer F.Cu) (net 9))
 (segment (start 104.4 117.6) (end 105.05 117.6) (width 0.25) (layer F.Cu) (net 9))
 (segment (start 106.8 118.9) (end 106.8 119.5) (width 0.25) (layer F.Cu) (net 10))
 (segment (start 106.8 118.55) (end 106.8 118.9) (width 0.25) (layer F.Cu) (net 10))
 (segment (start 105.05 116.8) (end 106.8 118.55) (width 0.25) (layer F.Cu) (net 10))
 (segment (start 104.4 116.8) (end 105.05 116.8) (width 0.25) (layer F.Cu) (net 10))
 (segment (start 104.4 116.3) (end 104.4 116.8) (width 0.25) (layer F.Cu) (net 10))
 (segment (start 104.4 115.9) (end 104.4 116.3) (width 0.25) (layer F.Cu) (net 10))
 (segment (start 100 111.5) (end 104.4 115.9) (width 0.25) (layer F.Cu) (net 10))
 (segment (start 103.40001 131.17499) (end 104.62501 131.17499) (width 0.25) (layer F.Cu) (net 3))
 (segment (start 103.075 131.5) (end 103.40001 131.17499) (width 0.25) (layer F.Cu) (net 3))
 (segment (start 103.075 132.2) (end 103.075 131.5) (width 0.25) (layer F.Cu) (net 3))
 (segment (start 106.3 129.5) (end 107.3 129.5) (width 0.25) (layer F.Cu) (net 3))
 (segment (start 104.62501 131.17499) (end 105.65 130.15) (width 0.25) (layer F.Cu) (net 3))
 (via (at 110 115.5) (size 0.8) (drill 0.4) (layers F.Cu B.Cu) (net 3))
 (via (at 119.5 115) (size 0.8) (drill 0.4) (layers F.Cu B.Cu) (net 3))
 (via (at 120 128) (size 0.8) (drill 0.4) (layers F.Cu B.Cu) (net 3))
 (via (at 110.5 127.5) (size 0.8) (drill 0.4) (layers F.Cu B.Cu) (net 3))
 (segment (start 105.65 130.15) (end 106.3 129.5) (width 0.25) (layer F.Cu) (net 3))
 (via (at 105.65 130.15) (size 0.8) (drill 0.4) (layers F.Cu B.Cu) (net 3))
 (via (at 105 112) (size 0.8) (drill 0.4) (layers F.Cu B.Cu) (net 3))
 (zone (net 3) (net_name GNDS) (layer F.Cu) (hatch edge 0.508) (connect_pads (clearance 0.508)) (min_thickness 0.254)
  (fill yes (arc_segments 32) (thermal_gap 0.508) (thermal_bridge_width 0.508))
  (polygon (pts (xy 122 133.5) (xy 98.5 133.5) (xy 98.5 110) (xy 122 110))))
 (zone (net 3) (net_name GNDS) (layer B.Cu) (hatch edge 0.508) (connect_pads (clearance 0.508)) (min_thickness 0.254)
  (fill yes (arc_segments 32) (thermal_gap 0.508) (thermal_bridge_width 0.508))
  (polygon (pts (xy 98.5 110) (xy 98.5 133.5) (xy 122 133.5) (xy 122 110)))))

